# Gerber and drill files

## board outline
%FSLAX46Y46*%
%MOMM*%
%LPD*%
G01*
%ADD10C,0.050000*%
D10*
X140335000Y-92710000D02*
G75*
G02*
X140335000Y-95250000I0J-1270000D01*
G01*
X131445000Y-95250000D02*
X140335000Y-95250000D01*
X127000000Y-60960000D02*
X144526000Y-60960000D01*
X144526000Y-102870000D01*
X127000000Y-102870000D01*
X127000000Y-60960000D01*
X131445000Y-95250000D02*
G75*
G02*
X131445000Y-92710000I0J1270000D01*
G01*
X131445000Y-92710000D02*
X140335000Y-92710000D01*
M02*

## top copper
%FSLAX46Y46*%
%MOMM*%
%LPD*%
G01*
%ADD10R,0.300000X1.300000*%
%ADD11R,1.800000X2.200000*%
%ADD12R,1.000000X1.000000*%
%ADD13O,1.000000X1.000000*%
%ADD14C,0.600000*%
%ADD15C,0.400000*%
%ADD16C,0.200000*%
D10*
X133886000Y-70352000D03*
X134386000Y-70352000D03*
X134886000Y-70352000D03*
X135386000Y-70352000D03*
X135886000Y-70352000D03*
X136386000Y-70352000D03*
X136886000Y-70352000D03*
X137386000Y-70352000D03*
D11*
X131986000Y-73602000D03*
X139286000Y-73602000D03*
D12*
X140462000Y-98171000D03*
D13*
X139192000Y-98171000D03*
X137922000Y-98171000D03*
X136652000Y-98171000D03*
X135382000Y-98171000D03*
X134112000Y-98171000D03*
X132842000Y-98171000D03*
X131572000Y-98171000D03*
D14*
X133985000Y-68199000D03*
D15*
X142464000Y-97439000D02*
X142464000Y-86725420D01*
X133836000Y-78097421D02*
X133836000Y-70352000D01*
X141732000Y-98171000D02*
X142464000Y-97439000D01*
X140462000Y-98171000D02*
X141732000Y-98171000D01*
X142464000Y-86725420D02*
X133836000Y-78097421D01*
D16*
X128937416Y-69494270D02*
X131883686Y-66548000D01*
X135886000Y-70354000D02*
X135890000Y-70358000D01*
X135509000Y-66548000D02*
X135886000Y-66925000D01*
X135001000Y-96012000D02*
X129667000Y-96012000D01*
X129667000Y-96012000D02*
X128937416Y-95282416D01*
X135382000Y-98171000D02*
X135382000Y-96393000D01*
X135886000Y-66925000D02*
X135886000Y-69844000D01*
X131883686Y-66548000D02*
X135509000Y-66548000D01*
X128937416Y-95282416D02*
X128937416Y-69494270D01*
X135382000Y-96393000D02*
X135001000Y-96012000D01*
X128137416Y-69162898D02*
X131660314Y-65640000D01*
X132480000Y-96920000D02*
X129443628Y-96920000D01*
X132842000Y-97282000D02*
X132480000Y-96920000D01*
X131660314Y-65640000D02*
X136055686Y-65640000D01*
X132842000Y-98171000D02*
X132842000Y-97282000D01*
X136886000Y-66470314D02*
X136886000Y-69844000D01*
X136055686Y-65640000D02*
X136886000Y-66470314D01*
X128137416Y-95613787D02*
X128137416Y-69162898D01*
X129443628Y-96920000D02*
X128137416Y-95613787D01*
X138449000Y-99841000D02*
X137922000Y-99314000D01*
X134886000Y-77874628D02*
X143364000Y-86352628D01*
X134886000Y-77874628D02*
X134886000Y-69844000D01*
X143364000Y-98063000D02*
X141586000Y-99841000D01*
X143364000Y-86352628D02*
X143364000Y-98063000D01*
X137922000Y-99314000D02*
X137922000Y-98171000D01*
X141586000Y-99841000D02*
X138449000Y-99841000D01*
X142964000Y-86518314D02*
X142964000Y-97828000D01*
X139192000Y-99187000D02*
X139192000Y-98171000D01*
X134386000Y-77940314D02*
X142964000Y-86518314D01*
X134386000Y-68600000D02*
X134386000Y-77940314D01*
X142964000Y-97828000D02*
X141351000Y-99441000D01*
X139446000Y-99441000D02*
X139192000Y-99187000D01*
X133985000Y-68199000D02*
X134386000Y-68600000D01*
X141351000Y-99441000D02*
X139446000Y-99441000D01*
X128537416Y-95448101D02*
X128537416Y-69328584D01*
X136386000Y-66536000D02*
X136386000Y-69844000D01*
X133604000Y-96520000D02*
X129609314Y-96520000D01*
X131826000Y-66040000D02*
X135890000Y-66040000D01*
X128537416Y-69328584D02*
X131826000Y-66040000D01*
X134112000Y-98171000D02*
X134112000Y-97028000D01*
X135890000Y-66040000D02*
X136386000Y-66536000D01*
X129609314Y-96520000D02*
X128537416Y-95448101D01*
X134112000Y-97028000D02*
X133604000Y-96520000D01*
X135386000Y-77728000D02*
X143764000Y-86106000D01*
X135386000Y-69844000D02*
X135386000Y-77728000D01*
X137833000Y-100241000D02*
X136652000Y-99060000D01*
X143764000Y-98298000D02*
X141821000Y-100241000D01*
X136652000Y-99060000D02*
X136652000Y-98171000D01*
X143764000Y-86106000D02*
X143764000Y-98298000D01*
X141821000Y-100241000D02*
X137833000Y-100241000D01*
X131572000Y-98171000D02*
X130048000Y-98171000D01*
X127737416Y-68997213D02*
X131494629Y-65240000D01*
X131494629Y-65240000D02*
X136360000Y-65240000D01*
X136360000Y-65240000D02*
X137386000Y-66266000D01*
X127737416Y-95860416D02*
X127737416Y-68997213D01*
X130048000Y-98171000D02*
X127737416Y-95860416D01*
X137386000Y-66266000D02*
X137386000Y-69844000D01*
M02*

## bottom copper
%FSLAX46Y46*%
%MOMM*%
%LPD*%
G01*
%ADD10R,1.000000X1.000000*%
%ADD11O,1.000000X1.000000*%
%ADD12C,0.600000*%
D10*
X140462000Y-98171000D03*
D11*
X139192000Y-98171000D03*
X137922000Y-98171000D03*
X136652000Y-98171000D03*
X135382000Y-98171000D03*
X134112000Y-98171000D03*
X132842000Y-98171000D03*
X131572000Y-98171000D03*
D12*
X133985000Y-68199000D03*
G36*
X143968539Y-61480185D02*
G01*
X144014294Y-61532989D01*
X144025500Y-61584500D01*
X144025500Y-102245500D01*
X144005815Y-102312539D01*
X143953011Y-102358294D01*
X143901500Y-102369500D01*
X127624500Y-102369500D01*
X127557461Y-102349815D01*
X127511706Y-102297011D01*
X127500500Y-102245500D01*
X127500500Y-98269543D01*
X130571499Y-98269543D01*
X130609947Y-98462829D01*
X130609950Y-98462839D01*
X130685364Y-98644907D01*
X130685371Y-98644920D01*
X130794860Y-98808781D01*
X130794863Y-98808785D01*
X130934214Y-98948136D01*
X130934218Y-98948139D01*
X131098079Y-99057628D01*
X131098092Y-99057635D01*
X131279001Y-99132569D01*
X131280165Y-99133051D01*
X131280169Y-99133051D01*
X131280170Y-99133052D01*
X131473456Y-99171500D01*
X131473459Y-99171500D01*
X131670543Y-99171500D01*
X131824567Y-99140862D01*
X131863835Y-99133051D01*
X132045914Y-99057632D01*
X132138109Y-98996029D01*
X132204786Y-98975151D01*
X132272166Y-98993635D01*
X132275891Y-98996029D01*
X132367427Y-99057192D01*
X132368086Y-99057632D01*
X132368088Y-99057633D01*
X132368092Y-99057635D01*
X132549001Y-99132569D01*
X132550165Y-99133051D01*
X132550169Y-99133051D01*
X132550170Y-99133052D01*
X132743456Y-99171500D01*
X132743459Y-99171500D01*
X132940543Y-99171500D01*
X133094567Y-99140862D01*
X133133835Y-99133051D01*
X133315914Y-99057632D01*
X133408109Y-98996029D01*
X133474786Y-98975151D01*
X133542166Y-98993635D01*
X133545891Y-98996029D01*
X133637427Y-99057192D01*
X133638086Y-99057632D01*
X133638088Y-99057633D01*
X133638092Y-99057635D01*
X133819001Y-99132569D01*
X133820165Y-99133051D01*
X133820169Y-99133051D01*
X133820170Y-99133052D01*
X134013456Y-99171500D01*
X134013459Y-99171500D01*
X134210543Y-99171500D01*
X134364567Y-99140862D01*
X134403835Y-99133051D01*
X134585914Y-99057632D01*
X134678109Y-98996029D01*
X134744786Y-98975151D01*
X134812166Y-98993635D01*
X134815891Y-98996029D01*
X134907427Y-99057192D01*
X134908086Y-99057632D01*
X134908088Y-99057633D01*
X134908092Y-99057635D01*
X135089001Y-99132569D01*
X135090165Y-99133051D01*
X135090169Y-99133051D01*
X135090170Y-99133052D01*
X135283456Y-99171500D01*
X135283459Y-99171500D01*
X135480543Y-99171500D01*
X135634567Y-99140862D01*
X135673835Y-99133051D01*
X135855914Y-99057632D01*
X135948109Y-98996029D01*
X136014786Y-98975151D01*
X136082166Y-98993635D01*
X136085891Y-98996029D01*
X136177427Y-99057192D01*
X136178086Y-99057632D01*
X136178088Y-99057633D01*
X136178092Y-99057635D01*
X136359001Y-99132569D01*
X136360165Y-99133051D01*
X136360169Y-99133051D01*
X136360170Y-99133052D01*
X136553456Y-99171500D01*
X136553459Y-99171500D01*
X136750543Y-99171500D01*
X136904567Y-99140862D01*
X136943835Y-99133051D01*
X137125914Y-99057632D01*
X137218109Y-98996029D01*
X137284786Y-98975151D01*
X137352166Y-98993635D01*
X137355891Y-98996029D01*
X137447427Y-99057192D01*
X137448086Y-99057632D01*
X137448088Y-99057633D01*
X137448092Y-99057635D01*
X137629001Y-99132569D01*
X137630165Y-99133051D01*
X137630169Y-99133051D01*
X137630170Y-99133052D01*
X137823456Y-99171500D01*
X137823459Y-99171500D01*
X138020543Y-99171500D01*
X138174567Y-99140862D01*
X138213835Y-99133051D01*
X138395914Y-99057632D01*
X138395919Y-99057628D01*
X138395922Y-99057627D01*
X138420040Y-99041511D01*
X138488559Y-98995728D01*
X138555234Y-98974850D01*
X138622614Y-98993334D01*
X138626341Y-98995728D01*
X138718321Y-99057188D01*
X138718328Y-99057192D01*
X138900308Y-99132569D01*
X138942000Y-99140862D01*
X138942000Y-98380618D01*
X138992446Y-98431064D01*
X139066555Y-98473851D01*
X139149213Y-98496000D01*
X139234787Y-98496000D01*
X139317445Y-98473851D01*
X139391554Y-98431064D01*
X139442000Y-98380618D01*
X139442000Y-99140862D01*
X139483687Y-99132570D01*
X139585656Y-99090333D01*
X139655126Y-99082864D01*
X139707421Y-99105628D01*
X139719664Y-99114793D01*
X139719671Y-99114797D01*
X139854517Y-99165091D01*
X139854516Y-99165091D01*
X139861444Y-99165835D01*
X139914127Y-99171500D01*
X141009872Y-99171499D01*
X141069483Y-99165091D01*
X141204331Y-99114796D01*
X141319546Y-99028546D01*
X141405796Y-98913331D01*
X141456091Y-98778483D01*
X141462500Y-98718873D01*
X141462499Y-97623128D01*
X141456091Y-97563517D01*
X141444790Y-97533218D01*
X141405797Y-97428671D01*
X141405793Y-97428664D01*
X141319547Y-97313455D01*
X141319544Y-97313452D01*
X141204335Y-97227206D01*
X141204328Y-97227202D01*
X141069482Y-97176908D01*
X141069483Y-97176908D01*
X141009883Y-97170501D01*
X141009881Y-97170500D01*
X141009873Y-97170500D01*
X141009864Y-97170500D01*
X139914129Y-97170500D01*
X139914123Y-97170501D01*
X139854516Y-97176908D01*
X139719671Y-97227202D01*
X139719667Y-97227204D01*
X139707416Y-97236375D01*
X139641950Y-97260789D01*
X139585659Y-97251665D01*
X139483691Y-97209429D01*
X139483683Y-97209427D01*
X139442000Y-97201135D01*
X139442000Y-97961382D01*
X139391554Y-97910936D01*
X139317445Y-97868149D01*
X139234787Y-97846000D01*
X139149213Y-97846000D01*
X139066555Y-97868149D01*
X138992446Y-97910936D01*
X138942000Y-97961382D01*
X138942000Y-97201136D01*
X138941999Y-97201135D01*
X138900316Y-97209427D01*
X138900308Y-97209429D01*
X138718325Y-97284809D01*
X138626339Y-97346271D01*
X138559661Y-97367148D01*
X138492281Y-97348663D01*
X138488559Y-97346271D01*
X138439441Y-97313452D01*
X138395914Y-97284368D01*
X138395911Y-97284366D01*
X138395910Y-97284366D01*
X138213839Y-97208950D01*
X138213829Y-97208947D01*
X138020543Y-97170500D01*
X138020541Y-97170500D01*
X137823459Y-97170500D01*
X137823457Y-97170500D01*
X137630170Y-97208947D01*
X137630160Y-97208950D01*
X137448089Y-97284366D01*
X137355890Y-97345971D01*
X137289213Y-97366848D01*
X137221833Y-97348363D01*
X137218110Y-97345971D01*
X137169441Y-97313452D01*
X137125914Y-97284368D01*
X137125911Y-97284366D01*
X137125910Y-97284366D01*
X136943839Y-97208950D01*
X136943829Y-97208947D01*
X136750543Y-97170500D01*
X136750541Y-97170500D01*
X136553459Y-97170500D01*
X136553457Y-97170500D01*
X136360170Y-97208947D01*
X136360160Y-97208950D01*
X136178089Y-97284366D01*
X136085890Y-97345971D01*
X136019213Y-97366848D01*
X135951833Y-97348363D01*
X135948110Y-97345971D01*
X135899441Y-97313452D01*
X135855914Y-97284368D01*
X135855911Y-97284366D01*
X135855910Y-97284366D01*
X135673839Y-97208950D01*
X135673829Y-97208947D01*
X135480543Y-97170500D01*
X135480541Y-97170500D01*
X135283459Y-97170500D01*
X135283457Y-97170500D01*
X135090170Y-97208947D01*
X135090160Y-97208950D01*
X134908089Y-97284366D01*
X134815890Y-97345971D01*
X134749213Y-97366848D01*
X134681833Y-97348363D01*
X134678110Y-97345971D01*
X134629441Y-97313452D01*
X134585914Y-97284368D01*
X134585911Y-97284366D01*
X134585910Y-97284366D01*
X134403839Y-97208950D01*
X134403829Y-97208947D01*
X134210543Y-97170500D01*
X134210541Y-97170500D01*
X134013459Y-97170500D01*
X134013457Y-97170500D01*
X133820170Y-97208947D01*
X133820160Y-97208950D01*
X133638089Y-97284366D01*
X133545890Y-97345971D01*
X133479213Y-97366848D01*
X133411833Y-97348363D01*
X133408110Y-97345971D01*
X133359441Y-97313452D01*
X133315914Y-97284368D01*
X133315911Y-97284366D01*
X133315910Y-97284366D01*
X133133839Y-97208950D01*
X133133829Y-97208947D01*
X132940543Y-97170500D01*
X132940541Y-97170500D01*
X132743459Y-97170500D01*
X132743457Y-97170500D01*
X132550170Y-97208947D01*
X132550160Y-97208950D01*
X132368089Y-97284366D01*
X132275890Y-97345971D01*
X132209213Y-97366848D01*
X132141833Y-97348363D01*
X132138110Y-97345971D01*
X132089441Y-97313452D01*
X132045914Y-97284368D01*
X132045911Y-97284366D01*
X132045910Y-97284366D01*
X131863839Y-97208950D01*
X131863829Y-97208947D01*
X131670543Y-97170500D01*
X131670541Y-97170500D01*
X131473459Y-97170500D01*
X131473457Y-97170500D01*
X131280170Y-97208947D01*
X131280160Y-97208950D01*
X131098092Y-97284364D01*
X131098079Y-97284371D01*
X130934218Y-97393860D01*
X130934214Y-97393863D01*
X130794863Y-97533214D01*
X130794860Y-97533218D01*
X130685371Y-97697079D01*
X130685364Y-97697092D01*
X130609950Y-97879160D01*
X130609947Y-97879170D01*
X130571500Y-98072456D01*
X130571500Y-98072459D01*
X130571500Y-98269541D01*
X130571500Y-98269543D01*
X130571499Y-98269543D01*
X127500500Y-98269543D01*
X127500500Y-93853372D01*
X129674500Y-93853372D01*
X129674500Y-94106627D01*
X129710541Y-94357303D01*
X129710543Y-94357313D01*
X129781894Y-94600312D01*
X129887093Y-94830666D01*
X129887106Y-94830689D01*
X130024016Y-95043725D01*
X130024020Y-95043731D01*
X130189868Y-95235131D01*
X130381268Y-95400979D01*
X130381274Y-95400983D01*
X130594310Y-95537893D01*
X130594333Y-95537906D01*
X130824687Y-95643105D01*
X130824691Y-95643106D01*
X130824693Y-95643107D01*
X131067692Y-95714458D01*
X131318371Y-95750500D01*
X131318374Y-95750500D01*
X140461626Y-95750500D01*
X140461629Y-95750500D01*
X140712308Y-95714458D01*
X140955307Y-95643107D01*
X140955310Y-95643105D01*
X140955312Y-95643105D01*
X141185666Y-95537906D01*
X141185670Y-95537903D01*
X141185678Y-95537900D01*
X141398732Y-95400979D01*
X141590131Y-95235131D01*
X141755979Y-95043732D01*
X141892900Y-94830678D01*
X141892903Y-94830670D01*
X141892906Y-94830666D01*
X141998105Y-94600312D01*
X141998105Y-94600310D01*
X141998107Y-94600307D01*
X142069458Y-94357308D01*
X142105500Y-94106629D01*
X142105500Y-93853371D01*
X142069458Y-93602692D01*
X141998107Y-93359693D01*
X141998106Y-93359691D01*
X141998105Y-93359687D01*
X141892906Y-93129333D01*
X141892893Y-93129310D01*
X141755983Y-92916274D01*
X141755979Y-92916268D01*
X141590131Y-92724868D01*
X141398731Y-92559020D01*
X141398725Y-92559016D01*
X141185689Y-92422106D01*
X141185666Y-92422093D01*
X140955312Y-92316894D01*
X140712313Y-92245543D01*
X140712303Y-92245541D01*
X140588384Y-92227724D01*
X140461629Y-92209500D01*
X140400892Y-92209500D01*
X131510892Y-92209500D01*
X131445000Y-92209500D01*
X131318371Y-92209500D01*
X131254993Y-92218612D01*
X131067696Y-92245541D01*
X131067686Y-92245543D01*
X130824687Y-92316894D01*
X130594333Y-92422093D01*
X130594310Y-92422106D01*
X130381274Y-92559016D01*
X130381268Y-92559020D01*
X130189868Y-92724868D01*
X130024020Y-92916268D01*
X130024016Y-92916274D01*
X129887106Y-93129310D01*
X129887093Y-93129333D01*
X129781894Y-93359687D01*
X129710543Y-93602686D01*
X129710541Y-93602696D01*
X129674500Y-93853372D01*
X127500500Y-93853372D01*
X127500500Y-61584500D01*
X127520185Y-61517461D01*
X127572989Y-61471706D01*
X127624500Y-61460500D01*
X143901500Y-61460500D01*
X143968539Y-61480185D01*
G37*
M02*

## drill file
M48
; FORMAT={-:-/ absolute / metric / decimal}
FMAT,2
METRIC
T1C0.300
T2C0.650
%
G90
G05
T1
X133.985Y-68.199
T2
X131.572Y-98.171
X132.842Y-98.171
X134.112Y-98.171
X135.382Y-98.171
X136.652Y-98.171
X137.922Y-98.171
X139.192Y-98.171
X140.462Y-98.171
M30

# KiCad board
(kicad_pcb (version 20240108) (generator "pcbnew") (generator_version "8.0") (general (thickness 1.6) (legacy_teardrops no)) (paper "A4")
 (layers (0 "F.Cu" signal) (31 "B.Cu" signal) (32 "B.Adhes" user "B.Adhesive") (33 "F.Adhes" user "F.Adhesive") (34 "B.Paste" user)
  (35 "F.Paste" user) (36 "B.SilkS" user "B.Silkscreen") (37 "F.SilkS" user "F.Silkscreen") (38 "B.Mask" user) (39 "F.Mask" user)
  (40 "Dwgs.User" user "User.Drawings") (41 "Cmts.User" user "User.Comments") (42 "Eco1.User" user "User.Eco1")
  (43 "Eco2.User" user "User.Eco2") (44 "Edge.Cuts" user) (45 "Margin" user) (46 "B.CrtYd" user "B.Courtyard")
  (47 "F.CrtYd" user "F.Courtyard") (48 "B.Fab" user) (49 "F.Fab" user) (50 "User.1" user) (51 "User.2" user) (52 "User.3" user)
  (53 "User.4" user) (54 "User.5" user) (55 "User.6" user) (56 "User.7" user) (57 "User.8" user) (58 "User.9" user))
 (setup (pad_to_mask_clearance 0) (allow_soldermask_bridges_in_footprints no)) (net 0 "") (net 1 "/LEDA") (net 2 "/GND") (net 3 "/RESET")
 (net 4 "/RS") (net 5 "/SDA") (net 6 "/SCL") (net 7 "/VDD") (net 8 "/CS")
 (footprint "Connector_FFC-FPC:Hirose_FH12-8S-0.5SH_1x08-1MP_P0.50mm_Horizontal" (layer "F.Cu") (at 135.636 72.202)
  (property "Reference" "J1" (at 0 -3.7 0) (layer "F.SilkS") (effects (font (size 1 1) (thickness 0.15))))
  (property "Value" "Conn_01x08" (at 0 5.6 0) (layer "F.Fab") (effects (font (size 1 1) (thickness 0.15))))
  (pad "1" smd rect (at -1.75 -1.85) (size 0.3 1.3) (layers "F.Cu" "F.Paste" "F.Mask") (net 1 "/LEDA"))
  (pad "2" smd rect (at -1.25 -1.85) (size 0.3 1.3) (layers "F.Cu" "F.Paste" "F.Mask") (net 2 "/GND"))
  (pad "3" smd rect (at -0.75 -1.85) (size 0.3 1.3) (layers "F.Cu" "F.Paste" "F.Mask") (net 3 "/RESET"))
  (pad "4" smd rect (at -0.25 -1.85) (size 0.3 1.3) (layers "F.Cu" "F.Paste" "F.Mask") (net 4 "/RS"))
  (pad "5" smd rect (at 0.25 -1.85) (size 0.3 1.3) (layers "F.Cu" "F.Paste" "F.Mask") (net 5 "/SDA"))
  (pad "6" smd rect (at 0.75 -1.85) (size 0.3 1.3) (layers "F.Cu" "F.Paste" "F.Mask") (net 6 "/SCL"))
  (pad "7" smd rect (at 1.25 -1.85) (size 0.3 1.3) (layers "F.Cu" "F.Paste" "F.Mask") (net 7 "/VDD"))
  (pad "8" smd rect (at 1.75 -1.85) (size 0.3 1.3) (layers "F.Cu" "F.Paste" "F.Mask") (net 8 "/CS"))
  (pad "MP" smd rect (at -3.65 1.4) (size 1.8 2.2) (layers "F.Cu" "F.Paste" "F.Mask"))
  (pad "MP" smd rect (at 3.65 1.4) (size 1.8 2.2) (layers "F.Cu" "F.Paste" "F.Mask")))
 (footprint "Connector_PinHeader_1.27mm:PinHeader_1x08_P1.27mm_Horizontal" (layer "F.Cu") (at 140.462 98.171 -90)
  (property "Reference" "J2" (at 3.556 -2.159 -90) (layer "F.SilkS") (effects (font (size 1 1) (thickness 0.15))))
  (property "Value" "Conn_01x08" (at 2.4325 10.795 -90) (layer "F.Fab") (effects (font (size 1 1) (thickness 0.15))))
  (pad "1" thru_hole rect (at 0 0 270) (size 1 1) (drill 0.65) (layers "*.Cu" "*.Mask") (remove_unused_layers no) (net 1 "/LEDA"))
  (pad "2" thru_hole oval (at 0 1.27 270) (size 1 1) (drill 0.65) (layers "*.Cu" "*.Mask") (remove_unused_layers no) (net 2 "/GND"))
  (pad "3" thru_hole oval (at 0 2.54 270) (size 1 1) (drill 0.65) (layers "*.Cu" "*.Mask") (remove_unused_layers no) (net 3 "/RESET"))
  (pad "4" thru_hole oval (at 0 3.81 270) (size 1 1) (drill 0.65) (layers "*.Cu" "*.Mask") (remove_unused_layers no) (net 4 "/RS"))
  (pad "5" thru_hole oval (at 0 5.08 270) (size 1 1) (drill 0.65) (layers "*.Cu" "*.Mask") (remove_unused_layers no) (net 5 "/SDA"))
  (pad "6" thru_hole oval (at 0 6.35 270) (size 1 1) (drill 0.65) (layers "*.Cu" "*.Mask") (remove_unused_layers no) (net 6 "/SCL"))
  (pad "7" thru_hole oval (at 0 7.62 270) (size 1 1) (drill 0.65) (layers "*.Cu" "*.Mask") (remove_unused_layers no) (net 7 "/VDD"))
  (pad "8" thru_hole oval (at 0 8.89 270) (size 1 1) (drill 0.65) (layers "*.Cu" "*.Mask") (remove_unused_layers no) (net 8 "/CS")))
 (gr_arc (start 140.335 92.71) (mid 141.605 93.98) (end 140.335 95.25) (stroke (width 0.05) (type default)) (layer "Edge.Cuts"))
 (gr_line (start 131.445 95.25) (end 140.335 95.25) (stroke (width 0.05) (type default)) (layer "Edge.Cuts"))
 (gr_rect (start 127 60.96) (end 144.526 102.87) (stroke (width 0.05) (type default)) (fill none) (layer "Edge.Cuts"))
 (gr_arc (start 131.445 95.25) (mid 130.175 93.98) (end 131.445 92.71) (stroke (width 0.05) (type default)) (layer "Edge.Cuts"))
 (gr_line (start 131.445 92.71) (end 140.335 92.71) (stroke (width 0.05) (type default)) (layer "Edge.Cuts"))
 (segment (start 142.464 97.439) (end 142.464 86.72542) (width 0.4) (layer "F.Cu") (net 1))
 (segment (start 133.836 78.097421) (end 133.836 70.352) (width 0.4) (layer "F.Cu") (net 1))
 (segment (start 141.732 98.171) (end 142.464 97.439) (width 0.4) (layer "F.Cu") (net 1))
 (segment (start 140.462 98.171) (end 141.732 98.171) (width 0.4) (layer "F.Cu") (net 1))
 (segment (start 142.464 86.72542) (end 133.836 78.097421) (width 0.4) (layer "F.Cu") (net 1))
 (segment (start 128.937416 69.49427) (end 131.883686 66.548) (width 0.2) (layer "F.Cu") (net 5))
 (segment (start 135.886 70.354) (end 135.89 70.358) (width 0.2) (layer "F.Cu") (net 5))
 (segment (start 135.509 66.548) (end 135.886 66.925) (width 0.2) (layer "F.Cu") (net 5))
 (segment (start 135.001 96.012) (end 129.667 96.012) (width 0.2) (layer "F.Cu") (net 5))
 (segment (start 129.667 96.012) (end 128.937416 95.282416) (width 0.2) (layer "F.Cu") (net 5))
 (segment (start 135.382 98.171) (end 135.382 96.393) (width 0.2) (layer "F.Cu") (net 5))
 (segment (start 135.886 66.925) (end 135.886 69.844) (width 0.2) (layer "F.Cu") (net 5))
 (segment (start 131.883686 66.548) (end 135.509 66.548) (width 0.2) (layer "F.Cu") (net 5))
 (segment (start 128.937416 95.282416) (end 128.937416 69.49427) (width 0.2) (layer "F.Cu") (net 5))
 (segment (start 135.382 96.393) (end 135.001 96.012) (width 0.2) (layer "F.Cu") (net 5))
 (segment (start 128.137416 69.162898) (end 131.660314 65.64) (width 0.2) (layer "F.Cu") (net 7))
 (segment (start 132.48 96.92) (end 129.443628 96.92) (width 0.2) (layer "F.Cu") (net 7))
 (segment (start 132.842 97.282) (end 132.48 96.92) (width 0.2) (layer "F.Cu") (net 7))
 (segment (start 131.660314 65.64) (end 136.055686 65.64) (width 0.2) (layer "F.Cu") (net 7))
 (segment (start 132.842 98.171) (end 132.842 97.282) (width 0.2) (layer "F.Cu") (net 7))
 (segment (start 136.886 66.470314) (end 136.886 69.844) (width 0.2) (layer "F.Cu") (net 7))
 (segment (start 136.055686 65.64) (end 136.886 66.470314) (width 0.2) (layer "F.Cu") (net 7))
 (segment (start 128.137416 95.613787) (end 128.137416 69.162898) (width 0.2) (layer "F.Cu") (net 7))
 (segment (start 129.443628 96.92) (end 128.137416 95.613787) (width 0.2) (layer "F.Cu") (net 7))
 (segment (start 138.449 99.841) (end 137.922 99.314) (width 0.2) (layer "F.Cu") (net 3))
 (segment (start 134.886 77.874628) (end 143.364 86.352628) (width 0.2) (layer "F.Cu") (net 3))
 (segment (start 134.886 77.874628) (end 134.886 69.844) (width 0.2) (layer "F.Cu") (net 3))
 (segment (start 143.364 98.063) (end 141.586 99.841) (width 0.2) (layer "F.Cu") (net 3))
 (segment (start 143.364 86.352628) (end 143.364 98.063) (width 0.2) (layer "F.Cu") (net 3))
 (segment (start 137.922 99.314) (end 137.922 98.171) (width 0.2) (layer "F.Cu") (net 3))
 (segment (start 141.586 99.841) (end 138.449 99.841) (width 0.2) (layer "F.Cu") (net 3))
 (segment (start 142.964 86.518314) (end 142.964 97.828) (width 0.2) (layer "F.Cu") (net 2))
 (segment (start 139.192 99.187) (end 139.192 98.171) (width 0.2) (layer "F.Cu") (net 2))
 (segment (start 134.386 77.940314) (end 142.964 86.518314) (width 0.2) (layer "F.Cu") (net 2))
 (segment (start 134.386 68.6) (end 134.386 77.940314) (width 0.2) (layer "F.Cu") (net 2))
 (segment (start 142.964 97.828) (end 141.351 99.441) (width 0.2) (layer "F.Cu") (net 2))
 (segment (start 139.446 99.441) (end 139.192 99.187) (width 0.2) (layer "F.Cu") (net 2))
 (segment (start 133.985 68.199) (end 134.386 68.6) (width 0.2) (layer "F.Cu") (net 2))
 (segment (start 141.351 99.441) (end 139.446 99.441) (width 0.2) (layer "F.Cu") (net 2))
 (via (at 133.985 68.199) (size 0.6) (drill 0.3) (layers "F.Cu" "B.Cu") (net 2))
 (segment (start 128.537416 95.448101) (end 128.537416 69.328584) (width 0.2) (layer "F.Cu") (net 6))
 (segment (start 136.386 66.536) (end 136.386 69.844) (width 0.2) (layer "F.Cu") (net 6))
 (segment (start 133.604 96.52) (end 129.609314 96.52) (width 0.2) (layer "F.Cu") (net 6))
 (segment (start 131.826 66.04) (end 135.89 66.04) (width 0.2) (layer "F.Cu") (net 6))
 (segment (start 128.537416 69.328584) (end 131.826 66.04) (width 0.2) (layer "F.Cu") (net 6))
 (segment (start 134.112 98.171) (end 134.112 97.028) (width 0.2) (layer "F.Cu") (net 6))
 (segment (start 135.89 66.04) (end 136.386 66.536) (width 0.2) (layer "F.Cu") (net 6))
 (segment (start 129.609314 96.52) (end 128.537416 95.448101) (width 0.2) (layer "F.Cu") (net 6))
 (segment (start 134.112 97.028) (end 133.604 96.52) (width 0.2) (layer "F.Cu") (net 6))
 (segment (start 135.386 77.728) (end 143.764 86.106) (width 0.2) (layer "F.Cu") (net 4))
 (segment (start 135.386 69.844) (end 135.386 77.728) (width 0.2) (layer "F.Cu") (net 4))
 (segment (start 137.833 100.241) (end 136.652 99.06) (width 0.2) (layer "F.Cu") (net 4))
 (segment (start 143.764 98.298) (end 141.821 100.241) (width 0.2) (layer "F.Cu") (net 4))
 (segment (start 136.652 99.06) (end 136.652 98.171) (width 0.2) (layer "F.Cu") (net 4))
 (segment (start 143.764 86.106) (end 143.764 98.298) (width 0.2) (layer "F.Cu") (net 4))
 (segment (start 141.821 100.241) (end 137.833 100.241) (width 0.2) (layer "F.Cu") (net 4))
 (segment (start 131.572 98.171) (end 130.048 98.171) (width 0.2) (layer "F.Cu") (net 8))
 (segment (start 127.737416 68.997213) (end 131.494629 65.24) (width 0.2) (layer "F.Cu") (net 8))
 (segment (start 131.494629 65.24) (end 136.36 65.24) (width 0.2) (layer "F.Cu") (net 8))
 (segment (start 136.36 65.24) (end 137.386 66.266) (width 0.2) (layer "F.Cu") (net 8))
 (segment (start 127.737416 95.860416) (end 127.737416 68.997213) (width 0.2) (layer "F.Cu") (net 8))
 (segment (start 130.048 98.171) (end 127.737416 95.860416) (width 0.2) (layer "F.Cu") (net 8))
 (segment (start 137.386 66.266) (end 137.386 69.844) (width 0.2) (layer "F.Cu") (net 8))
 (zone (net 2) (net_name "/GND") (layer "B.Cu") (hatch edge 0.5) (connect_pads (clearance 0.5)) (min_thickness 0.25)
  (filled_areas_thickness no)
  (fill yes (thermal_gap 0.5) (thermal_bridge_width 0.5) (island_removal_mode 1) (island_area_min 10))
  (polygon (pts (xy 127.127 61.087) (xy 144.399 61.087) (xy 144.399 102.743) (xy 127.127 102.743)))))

